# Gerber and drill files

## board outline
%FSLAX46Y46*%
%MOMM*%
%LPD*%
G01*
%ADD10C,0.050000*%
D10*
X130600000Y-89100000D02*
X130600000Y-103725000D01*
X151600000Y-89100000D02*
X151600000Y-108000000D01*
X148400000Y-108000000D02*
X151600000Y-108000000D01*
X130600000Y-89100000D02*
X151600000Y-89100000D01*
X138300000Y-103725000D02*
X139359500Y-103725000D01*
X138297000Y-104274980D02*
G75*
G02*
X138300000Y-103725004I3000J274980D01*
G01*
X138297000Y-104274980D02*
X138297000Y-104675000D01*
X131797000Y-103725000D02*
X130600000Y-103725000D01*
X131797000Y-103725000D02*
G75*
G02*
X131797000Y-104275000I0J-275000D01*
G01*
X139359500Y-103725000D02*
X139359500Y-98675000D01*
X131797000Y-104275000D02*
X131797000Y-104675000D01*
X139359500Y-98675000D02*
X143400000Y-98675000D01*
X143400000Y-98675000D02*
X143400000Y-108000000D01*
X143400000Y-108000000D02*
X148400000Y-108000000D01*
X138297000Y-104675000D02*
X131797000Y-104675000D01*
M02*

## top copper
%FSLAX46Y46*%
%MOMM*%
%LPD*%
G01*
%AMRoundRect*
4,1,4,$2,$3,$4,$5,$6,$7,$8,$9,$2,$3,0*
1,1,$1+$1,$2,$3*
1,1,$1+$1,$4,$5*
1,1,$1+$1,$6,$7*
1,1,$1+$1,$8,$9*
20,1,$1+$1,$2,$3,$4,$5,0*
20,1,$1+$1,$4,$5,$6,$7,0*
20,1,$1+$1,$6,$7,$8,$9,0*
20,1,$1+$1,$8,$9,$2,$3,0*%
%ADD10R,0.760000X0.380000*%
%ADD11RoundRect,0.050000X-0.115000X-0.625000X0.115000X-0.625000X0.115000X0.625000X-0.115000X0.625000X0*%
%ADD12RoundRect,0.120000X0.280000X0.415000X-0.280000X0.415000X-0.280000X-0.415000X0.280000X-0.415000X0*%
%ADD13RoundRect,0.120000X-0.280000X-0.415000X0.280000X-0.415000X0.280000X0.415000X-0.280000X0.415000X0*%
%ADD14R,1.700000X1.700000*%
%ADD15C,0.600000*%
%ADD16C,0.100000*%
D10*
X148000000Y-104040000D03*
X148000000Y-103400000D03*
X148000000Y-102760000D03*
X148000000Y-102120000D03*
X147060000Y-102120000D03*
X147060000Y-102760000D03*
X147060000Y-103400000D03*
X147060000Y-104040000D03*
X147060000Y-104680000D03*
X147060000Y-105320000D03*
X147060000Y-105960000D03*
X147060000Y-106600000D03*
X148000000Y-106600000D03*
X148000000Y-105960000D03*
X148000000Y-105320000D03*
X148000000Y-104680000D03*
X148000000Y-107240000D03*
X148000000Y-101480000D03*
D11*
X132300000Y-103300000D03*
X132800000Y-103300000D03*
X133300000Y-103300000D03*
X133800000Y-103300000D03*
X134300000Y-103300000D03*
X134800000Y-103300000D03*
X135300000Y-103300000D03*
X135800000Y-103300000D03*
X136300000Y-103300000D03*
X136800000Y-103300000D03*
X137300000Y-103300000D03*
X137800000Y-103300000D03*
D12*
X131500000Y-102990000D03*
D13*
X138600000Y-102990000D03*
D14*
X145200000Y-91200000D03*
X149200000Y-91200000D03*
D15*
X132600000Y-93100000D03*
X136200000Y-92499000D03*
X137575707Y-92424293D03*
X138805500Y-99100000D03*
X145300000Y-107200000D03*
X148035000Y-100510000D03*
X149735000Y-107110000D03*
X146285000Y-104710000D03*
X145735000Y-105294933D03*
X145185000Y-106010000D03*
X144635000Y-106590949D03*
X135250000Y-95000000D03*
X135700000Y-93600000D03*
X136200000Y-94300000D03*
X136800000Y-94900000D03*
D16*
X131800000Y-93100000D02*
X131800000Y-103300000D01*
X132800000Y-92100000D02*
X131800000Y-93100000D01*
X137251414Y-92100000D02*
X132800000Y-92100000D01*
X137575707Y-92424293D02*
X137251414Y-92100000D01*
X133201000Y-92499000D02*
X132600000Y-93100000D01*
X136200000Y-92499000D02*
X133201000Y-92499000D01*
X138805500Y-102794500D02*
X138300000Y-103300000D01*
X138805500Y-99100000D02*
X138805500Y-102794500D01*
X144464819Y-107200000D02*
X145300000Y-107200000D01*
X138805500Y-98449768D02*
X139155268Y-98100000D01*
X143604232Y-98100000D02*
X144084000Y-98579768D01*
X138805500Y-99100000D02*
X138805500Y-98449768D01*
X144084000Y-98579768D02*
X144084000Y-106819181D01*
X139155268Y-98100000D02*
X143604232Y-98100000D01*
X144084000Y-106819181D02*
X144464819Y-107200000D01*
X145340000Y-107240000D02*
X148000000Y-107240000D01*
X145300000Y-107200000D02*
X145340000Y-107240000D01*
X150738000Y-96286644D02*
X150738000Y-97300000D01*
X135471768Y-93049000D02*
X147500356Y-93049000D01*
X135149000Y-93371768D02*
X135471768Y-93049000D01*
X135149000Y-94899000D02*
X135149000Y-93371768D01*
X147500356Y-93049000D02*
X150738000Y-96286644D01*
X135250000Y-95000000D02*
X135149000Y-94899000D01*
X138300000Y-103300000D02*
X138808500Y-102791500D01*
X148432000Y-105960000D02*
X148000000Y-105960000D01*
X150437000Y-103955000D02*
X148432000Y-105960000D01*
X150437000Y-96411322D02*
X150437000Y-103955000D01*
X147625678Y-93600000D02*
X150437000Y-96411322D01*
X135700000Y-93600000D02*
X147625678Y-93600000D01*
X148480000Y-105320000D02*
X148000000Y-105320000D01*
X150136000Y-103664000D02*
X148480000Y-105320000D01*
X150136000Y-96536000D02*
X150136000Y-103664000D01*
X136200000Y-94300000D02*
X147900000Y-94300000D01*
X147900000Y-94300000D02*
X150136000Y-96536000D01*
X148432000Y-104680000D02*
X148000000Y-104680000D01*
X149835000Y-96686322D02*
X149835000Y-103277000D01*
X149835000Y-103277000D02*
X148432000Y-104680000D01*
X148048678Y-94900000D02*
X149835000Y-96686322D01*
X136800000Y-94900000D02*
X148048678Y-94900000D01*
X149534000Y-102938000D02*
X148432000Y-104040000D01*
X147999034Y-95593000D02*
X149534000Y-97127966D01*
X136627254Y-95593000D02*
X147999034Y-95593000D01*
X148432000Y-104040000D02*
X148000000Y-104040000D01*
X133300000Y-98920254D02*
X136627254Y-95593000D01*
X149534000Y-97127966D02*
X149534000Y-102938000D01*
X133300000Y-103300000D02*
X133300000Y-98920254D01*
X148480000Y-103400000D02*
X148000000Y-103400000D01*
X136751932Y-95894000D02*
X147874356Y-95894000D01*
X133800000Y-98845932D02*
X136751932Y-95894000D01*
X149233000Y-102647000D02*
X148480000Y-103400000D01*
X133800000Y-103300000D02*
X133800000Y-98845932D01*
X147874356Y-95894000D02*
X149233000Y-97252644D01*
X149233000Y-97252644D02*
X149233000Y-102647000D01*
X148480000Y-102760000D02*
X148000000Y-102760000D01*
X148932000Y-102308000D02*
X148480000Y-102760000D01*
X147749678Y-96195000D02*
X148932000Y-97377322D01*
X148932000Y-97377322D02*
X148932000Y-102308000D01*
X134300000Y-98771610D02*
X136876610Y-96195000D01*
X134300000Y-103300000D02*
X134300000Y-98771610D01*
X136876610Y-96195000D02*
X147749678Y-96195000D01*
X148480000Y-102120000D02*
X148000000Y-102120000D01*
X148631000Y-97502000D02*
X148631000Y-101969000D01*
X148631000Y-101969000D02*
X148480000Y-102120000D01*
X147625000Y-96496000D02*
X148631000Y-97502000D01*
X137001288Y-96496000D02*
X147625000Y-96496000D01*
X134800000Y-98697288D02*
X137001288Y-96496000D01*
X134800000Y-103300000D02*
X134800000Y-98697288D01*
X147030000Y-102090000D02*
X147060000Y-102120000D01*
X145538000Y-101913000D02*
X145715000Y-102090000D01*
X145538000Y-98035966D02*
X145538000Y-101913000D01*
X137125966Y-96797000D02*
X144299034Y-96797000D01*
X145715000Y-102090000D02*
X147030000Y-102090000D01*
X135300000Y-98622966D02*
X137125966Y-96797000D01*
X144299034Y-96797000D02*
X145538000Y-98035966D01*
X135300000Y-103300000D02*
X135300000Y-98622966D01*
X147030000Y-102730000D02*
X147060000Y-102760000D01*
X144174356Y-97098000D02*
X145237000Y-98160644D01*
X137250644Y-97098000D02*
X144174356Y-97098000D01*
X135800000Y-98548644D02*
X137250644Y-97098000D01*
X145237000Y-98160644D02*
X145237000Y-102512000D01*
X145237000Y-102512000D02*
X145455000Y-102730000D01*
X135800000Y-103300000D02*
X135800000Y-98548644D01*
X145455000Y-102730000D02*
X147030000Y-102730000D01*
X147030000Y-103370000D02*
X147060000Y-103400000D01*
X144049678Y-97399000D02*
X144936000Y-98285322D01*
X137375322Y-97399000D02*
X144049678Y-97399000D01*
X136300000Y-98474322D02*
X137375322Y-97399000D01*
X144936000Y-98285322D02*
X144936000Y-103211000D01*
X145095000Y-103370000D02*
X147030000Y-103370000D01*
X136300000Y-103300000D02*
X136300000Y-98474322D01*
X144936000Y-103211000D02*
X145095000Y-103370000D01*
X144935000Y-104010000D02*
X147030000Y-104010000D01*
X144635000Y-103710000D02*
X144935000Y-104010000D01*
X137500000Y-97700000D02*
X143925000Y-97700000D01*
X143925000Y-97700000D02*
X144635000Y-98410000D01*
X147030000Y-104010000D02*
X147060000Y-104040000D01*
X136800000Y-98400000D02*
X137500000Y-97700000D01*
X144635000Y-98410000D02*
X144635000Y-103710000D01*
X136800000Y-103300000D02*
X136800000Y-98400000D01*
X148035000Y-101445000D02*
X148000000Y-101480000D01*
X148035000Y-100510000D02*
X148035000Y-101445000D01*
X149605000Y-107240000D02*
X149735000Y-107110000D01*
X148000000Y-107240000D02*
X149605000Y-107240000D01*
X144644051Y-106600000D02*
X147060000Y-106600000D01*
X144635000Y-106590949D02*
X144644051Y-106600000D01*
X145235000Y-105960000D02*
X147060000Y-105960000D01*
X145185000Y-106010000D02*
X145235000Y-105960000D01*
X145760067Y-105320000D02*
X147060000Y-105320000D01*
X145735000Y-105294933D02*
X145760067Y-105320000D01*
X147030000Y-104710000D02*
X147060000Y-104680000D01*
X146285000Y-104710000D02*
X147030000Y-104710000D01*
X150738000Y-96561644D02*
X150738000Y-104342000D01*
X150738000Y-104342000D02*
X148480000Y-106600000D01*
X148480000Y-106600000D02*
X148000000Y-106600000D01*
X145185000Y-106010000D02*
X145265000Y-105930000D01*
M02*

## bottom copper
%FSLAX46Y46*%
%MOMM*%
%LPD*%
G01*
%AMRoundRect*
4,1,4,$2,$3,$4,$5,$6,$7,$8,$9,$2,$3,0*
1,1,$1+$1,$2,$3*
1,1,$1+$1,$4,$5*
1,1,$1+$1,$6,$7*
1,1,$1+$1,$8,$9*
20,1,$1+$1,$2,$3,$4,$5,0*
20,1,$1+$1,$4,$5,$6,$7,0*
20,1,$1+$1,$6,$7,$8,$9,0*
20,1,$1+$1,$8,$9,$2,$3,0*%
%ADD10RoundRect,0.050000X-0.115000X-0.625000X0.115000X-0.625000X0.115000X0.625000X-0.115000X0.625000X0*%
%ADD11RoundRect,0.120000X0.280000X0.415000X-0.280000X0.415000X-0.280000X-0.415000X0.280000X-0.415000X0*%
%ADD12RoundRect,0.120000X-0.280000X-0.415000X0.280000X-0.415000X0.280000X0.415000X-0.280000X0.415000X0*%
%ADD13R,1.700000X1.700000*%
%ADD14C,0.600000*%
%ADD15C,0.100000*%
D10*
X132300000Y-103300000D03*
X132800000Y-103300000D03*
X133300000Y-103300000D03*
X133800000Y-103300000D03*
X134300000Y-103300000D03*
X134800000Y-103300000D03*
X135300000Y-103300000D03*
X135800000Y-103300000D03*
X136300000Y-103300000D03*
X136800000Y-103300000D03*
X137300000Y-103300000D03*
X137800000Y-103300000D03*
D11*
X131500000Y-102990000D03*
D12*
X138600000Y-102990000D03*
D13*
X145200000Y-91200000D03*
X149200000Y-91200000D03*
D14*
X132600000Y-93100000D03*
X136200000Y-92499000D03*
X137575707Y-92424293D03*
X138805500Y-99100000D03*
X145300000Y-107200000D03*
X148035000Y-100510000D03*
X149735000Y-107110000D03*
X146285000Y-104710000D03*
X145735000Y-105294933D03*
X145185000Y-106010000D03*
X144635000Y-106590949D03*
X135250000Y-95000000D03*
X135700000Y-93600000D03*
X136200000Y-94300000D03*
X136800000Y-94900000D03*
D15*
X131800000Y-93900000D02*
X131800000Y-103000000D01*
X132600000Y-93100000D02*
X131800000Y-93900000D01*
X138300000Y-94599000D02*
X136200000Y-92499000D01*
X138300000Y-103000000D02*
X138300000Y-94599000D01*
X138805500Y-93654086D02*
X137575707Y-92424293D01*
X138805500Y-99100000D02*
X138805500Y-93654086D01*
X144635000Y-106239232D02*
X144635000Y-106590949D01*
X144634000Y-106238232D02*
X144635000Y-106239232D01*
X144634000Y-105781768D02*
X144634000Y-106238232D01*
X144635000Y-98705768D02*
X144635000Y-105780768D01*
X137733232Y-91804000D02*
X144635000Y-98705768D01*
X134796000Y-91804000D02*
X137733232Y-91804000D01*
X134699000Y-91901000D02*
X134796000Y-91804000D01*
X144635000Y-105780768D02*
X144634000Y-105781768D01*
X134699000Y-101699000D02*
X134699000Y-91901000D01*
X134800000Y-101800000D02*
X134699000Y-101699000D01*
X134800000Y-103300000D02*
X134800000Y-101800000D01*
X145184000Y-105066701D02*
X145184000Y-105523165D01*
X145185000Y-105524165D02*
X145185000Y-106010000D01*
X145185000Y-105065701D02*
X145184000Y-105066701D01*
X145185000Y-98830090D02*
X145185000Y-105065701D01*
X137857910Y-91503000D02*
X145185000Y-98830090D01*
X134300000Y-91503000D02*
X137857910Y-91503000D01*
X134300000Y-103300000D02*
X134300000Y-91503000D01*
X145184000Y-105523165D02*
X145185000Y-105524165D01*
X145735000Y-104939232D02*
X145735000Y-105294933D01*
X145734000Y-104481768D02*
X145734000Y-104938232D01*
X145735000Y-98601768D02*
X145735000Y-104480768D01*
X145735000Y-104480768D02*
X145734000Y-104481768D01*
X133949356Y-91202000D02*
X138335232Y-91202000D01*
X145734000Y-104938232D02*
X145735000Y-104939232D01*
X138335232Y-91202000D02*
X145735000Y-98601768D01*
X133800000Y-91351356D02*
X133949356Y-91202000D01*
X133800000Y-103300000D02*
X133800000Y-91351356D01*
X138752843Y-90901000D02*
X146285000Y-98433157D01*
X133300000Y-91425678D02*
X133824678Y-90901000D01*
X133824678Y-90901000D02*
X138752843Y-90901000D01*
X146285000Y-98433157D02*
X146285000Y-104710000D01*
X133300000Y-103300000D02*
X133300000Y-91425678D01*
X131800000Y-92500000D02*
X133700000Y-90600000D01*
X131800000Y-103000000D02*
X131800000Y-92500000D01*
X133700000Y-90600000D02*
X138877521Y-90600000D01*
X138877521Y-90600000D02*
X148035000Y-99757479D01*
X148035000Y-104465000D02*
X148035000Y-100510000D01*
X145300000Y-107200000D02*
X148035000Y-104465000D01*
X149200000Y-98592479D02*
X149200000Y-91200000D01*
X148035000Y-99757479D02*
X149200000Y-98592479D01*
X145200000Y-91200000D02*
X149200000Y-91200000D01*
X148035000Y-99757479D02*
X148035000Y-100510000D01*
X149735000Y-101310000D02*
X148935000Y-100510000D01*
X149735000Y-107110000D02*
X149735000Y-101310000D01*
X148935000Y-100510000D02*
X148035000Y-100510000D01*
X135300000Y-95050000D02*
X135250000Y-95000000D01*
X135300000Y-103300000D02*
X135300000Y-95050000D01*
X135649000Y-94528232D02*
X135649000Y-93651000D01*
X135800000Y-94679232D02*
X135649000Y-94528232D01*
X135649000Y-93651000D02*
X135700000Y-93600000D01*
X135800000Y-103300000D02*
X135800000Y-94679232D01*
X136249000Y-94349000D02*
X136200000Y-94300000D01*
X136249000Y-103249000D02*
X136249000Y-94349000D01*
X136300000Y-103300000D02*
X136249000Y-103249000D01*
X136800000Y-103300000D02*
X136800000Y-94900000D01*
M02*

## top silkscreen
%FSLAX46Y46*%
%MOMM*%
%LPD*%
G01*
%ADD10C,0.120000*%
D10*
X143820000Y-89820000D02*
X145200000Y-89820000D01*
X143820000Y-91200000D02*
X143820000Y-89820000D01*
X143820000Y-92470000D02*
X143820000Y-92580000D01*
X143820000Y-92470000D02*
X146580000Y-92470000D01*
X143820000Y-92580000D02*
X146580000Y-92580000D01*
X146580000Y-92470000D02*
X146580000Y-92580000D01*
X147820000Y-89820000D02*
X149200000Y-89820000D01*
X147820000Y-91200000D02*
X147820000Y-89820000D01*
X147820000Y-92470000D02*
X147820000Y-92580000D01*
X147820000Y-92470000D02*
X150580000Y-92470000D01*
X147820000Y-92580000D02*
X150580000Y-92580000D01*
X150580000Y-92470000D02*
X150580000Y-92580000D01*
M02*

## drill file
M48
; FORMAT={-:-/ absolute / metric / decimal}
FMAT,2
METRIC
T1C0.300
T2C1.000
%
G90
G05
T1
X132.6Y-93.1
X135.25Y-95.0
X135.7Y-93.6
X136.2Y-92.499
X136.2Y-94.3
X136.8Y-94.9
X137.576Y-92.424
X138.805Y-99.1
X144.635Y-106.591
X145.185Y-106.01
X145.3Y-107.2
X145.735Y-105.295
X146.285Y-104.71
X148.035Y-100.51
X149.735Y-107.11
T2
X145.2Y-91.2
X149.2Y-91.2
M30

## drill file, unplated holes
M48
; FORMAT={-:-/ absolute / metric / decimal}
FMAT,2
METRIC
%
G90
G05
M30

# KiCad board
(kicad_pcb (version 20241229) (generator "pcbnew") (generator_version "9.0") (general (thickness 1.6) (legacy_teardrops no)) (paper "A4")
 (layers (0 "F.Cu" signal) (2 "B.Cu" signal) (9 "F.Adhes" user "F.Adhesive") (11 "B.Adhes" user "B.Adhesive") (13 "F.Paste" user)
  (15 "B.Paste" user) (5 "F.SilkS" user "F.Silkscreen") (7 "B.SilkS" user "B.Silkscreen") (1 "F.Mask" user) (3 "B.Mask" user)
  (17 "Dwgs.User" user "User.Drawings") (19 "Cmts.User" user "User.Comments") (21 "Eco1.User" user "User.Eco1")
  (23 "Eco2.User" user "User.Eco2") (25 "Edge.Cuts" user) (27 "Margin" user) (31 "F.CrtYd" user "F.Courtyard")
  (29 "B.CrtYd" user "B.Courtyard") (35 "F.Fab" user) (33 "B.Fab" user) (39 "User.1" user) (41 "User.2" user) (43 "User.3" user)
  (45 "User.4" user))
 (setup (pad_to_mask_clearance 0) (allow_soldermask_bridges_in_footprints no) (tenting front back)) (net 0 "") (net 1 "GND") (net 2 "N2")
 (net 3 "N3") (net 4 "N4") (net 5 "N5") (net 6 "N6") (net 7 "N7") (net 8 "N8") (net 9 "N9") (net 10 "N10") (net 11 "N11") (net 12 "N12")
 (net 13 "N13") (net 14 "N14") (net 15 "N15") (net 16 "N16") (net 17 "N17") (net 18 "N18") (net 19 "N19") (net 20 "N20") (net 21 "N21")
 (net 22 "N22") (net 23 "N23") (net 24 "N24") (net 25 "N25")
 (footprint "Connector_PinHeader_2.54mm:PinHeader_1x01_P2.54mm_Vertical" (layer "F.Cu") (at 149.2 91.2)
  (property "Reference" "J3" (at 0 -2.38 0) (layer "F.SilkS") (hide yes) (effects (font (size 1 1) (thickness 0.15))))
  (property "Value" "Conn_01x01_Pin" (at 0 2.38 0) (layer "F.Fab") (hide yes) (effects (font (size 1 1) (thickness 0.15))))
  (fp_line (start -1.38 -1.38) (end 0 -1.38) (stroke (width 0.12) (type solid)) (layer "F.SilkS"))
  (fp_line (start -1.38 0) (end -1.38 -1.38) (stroke (width 0.12) (type solid)) (layer "F.SilkS"))
  (fp_line (start -1.38 1.27) (end -1.38 1.38) (stroke (width 0.12) (type solid)) (layer "F.SilkS"))
  (fp_line (start -1.38 1.27) (end 1.38 1.27) (stroke (width 0.12) (type solid)) (layer "F.SilkS"))
  (fp_line (start -1.38 1.38) (end 1.38 1.38) (stroke (width 0.12) (type solid)) (layer "F.SilkS"))
  (fp_line (start 1.38 1.27) (end 1.38 1.38) (stroke (width 0.12) (type solid)) (layer "F.SilkS"))
  (pad "1" thru_hole rect (at 0 0) (size 1.7 1.7) (drill 1) (layers "*.Cu" "*.Mask") (remove_unused_layers no) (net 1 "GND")))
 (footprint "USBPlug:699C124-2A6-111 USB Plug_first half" (layer "F.Cu") (at 134.8 100.3)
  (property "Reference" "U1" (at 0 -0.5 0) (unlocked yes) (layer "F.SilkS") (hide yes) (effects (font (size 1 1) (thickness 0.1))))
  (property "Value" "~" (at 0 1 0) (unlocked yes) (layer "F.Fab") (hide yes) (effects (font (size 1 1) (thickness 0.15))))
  (pad "0" smd roundrect (at -2.5 3) (size 0.33 1.35) (layers "F.Cu" "F.Mask" "F.Paste") (roundrect_rratio 0.1515151515) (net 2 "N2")
   (thermal_bridge_angle 45))
  (pad "1" smd roundrect (at -2 3) (size 0.33 1.35) (layers "F.Cu" "F.Mask" "F.Paste") (roundrect_rratio 0.1515151515) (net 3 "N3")
   (thermal_bridge_angle 45))
  (pad "2" smd roundrect (at -1.5 3) (size 0.33 1.35) (layers "F.Cu" "F.Mask" "F.Paste") (roundrect_rratio 0.1515151515) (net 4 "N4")
   (thermal_bridge_angle 45))
  (pad "3" smd roundrect (at -1 3) (size 0.33 1.35) (layers "F.Cu" "F.Mask" "F.Paste") (roundrect_rratio 0.1515151515) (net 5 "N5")
   (thermal_bridge_angle 45))
  (pad "4" smd roundrect (at -0.5 3) (size 0.33 1.35) (layers "F.Cu" "F.Mask" "F.Paste") (roundrect_rratio 0.1515151515) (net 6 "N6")
   (thermal_bridge_angle 45))
  (pad "5" smd roundrect (at 0 3) (size 0.33 1.35) (layers "F.Cu" "F.Mask" "F.Paste") (roundrect_rratio 0.1515151515) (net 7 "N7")
   (thermal_bridge_angle 45))
  (pad "6" smd roundrect (at 0.5 3) (size 0.33 1.35) (layers "F.Cu" "F.Mask" "F.Paste") (roundrect_rratio 0.1515151515) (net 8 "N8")
   (thermal_bridge_angle 45))
  (pad "7" smd roundrect (at 1 3) (size 0.33 1.35) (layers "F.Cu" "F.Mask" "F.Paste") (roundrect_rratio 0.1515151515) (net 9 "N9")
   (thermal_bridge_angle 45))
  (pad "8" smd roundrect (at 1.5 3) (size 0.33 1.35) (layers "F.Cu" "F.Mask" "F.Paste") (roundrect_rratio 0.1515151515) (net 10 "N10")
   (thermal_bridge_angle 45))
  (pad "9" smd roundrect (at 2 3) (size 0.33 1.35) (layers "F.Cu" "F.Mask" "F.Paste") (roundrect_rratio 0.1515151515) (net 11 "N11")
   (thermal_bridge_angle 45))
  (pad "10" smd roundrect (at 2.5 3) (size 0.33 1.35) (layers "F.Cu" "F.Mask" "F.Paste") (roundrect_rratio 0.1515151515) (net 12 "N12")
   (thermal_bridge_angle 45))
  (pad "11" smd roundrect (at 3 3) (size 0.33 1.35) (layers "F.Cu" "F.Mask" "F.Paste") (roundrect_rratio 0.1515151515) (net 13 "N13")
   (thermal_bridge_angle 45))
  (pad "24" smd roundrect (at -3 3 180) (size 0.8 1.07) (drill (offset 0.3 0.31)) (layers "F.Cu" "F.Mask" "F.Paste") (roundrect_rratio 0.15)
   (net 1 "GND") (thermal_bridge_angle 45))
  (pad "25" smd roundrect (at 3.5 3) (size 0.8 1.07) (drill (offset 0.3 -0.31)) (layers "F.Cu" "F.Mask" "F.Paste") (roundrect_rratio 0.15)
   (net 1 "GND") (thermal_bridge_angle 45)))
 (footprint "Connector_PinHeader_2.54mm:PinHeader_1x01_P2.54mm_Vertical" (layer "F.Cu") (at 145.2 91.2)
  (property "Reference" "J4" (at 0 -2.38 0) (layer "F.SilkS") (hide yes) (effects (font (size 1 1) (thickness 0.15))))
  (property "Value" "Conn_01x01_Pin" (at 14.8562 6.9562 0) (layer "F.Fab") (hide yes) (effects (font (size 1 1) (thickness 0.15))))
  (fp_line (start -1.38 -1.38) (end 0 -1.38) (stroke (width 0.12) (type solid)) (layer "F.SilkS"))
  (fp_line (start -1.38 0) (end -1.38 -1.38) (stroke (width 0.12) (type solid)) (layer "F.SilkS"))
  (fp_line (start -1.38 1.27) (end -1.38 1.38) (stroke (width 0.12) (type solid)) (layer "F.SilkS"))
  (fp_line (start -1.38 1.27) (end 1.38 1.27) (stroke (width 0.12) (type solid)) (layer "F.SilkS"))
  (fp_line (start -1.38 1.38) (end 1.38 1.38) (stroke (width 0.12) (type solid)) (layer "F.SilkS"))
  (fp_line (start 1.38 1.27) (end 1.38 1.38) (stroke (width 0.12) (type solid)) (layer "F.SilkS"))
  (pad "1" thru_hole rect (at 0 0) (size 1.7 1.7) (drill 1) (layers "*.Cu" "*.Mask") (remove_unused_layers no) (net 1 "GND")))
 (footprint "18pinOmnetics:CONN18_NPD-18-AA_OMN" (layer "F.Cu") (at 148.94 104.04 90)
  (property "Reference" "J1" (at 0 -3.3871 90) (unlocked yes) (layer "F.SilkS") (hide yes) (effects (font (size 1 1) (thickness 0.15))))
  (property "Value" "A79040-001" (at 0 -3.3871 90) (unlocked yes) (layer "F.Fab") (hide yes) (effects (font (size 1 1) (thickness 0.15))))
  (pad "0" smd rect (at 0 -0.94 90) (size 0.38 0.76) (layers "F.Cu" "F.Mask" "F.Paste") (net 4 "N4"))
  (pad "1" smd rect (at 0.64 -0.94 90) (size 0.38 0.76) (layers "F.Cu" "F.Mask" "F.Paste") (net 5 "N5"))
  (pad "2" smd rect (at 1.28 -0.94 90) (size 0.38 0.76) (layers "F.Cu" "F.Mask" "F.Paste") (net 6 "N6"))
  (pad "3" smd rect (at 1.92 -0.94 90) (size 0.38 0.76) (layers "F.Cu" "F.Mask" "F.Paste") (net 7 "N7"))
  (pad "4" smd rect (at 1.92 -1.88 90) (size 0.38 0.76) (layers "F.Cu" "F.Mask" "F.Paste") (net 8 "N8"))
  (pad "5" smd rect (at 1.28 -1.88 90) (size 0.38 0.76) (layers "F.Cu" "F.Mask" "F.Paste") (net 9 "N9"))
  (pad "6" smd rect (at 0.64 -1.88 90) (size 0.38 0.76) (layers "F.Cu" "F.Mask" "F.Paste") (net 10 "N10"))
  (pad "7" smd rect (at 0 -1.88 90) (size 0.38 0.76) (layers "F.Cu" "F.Mask" "F.Paste") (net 11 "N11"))
  (pad "8" smd rect (at -0.64 -1.88 90) (size 0.38 0.76) (layers "F.Cu" "F.Mask" "F.Paste") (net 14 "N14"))
  (pad "9" smd rect (at -1.28 -1.88 90) (size 0.38 0.76) (layers "F.Cu" "F.Mask" "F.Paste") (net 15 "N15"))
  (pad "10" smd rect (at -1.92 -1.88 90) (size 0.38 0.76) (layers "F.Cu" "F.Mask" "F.Paste") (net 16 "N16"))
  (pad "11" smd rect (at -2.56 -1.88 90) (size 0.38 0.76) (layers "F.Cu" "F.Mask" "F.Paste") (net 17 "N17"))
  (pad "12" smd rect (at -2.56 -0.94 90) (size 0.38 0.76) (layers "F.Cu" "F.Mask" "F.Paste") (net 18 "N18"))
  (pad "13" smd rect (at -1.92 -0.94 90) (size 0.38 0.76) (layers "F.Cu" "F.Mask" "F.Paste") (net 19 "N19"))
  (pad "14" smd rect (at -1.28 -0.94 90) (size 0.38 0.76) (layers "F.Cu" "F.Mask" "F.Paste") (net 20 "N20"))
  (pad "15" smd rect (at -0.64 -0.94 90) (size 0.38 0.76) (layers "F.Cu" "F.Mask" "F.Paste") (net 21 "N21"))
  (pad "16" smd rect (at -3.2 -0.94 90) (size 0.38 0.76) (layers "F.Cu" "F.Mask" "F.Paste") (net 1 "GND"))
  (pad "17" smd rect (at 2.56 -0.94 90) (size 0.38 0.76) (layers "F.Cu" "F.Mask" "F.Paste") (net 1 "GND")))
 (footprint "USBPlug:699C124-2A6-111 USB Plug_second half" (layer "B.Cu") (at 134.8 106.3)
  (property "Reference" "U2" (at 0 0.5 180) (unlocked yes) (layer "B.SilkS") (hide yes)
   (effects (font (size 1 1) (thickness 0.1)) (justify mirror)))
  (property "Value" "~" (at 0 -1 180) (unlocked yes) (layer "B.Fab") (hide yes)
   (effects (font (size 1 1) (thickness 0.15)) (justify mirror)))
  (pad "12" smd roundrect (at -2.5 -3) (size 0.33 1.35) (layers "B.Cu" "B.Mask" "B.Paste") (roundrect_rratio 0.1515151515) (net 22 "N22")
   (thermal_bridge_angle 45))
  (pad "13" smd roundrect (at -2 -3) (size 0.33 1.35) (layers "B.Cu" "B.Mask" "B.Paste") (roundrect_rratio 0.1515151515) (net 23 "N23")
   (thermal_bridge_angle 45))
  (pad "14" smd roundrect (at -1.5 -3) (size 0.33 1.35) (layers "B.Cu" "B.Mask" "B.Paste") (roundrect_rratio 0.1515151515) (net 14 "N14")
   (thermal_bridge_angle 45))
  (pad "15" smd roundrect (at -1 -3) (size 0.33 1.35) (layers "B.Cu" "B.Mask" "B.Paste") (roundrect_rratio 0.1515151515) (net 15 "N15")
   (thermal_bridge_angle 45))
  (pad "16" smd roundrect (at -0.5 -3) (size 0.33 1.35) (layers "B.Cu" "B.Mask" "B.Paste") (roundrect_rratio 0.1515151515) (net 16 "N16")
   (thermal_bridge_angle 45))
  (pad "17" smd roundrect (at 0 -3) (size 0.33 1.35) (layers "B.Cu" "B.Mask" "B.Paste") (roundrect_rratio 0.1515151515) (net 17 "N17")
   (thermal_bridge_angle 45))
  (pad "18" smd roundrect (at 0.5 -3) (size 0.33 1.35) (layers "B.Cu" "B.Mask" "B.Paste") (roundrect_rratio 0.1515151515) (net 18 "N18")
   (thermal_bridge_angle 45))
  (pad "19" smd roundrect (at 1 -3) (size 0.33 1.35) (layers "B.Cu" "B.Mask" "B.Paste") (roundrect_rratio 0.1515151515) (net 19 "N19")
   (thermal_bridge_angle 45))
  (pad "20" smd roundrect (at 1.5 -3) (size 0.33 1.35) (layers "B.Cu" "B.Mask" "B.Paste") (roundrect_rratio 0.1515151515) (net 20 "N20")
   (thermal_bridge_angle 45))
  (pad "21" smd roundrect (at 2 -3) (size 0.33 1.35) (layers "B.Cu" "B.Mask" "B.Paste") (roundrect_rratio 0.1515151515) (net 21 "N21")
   (thermal_bridge_angle 45))
  (pad "22" smd roundrect (at 2.5 -3) (size 0.33 1.35) (layers "B.Cu" "B.Mask" "B.Paste") (roundrect_rratio 0.1515151515) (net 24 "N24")
   (thermal_bridge_angle 45))
  (pad "23" smd roundrect (at 3 -3) (size 0.33 1.35) (layers "B.Cu" "B.Mask" "B.Paste") (roundrect_rratio 0.1515151515) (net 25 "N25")
   (thermal_bridge_angle 45))
  (pad "26" smd roundrect (at -3 -3.3 180) (size 0.8 1.07) (drill (offset 0.3 0.01)) (layers "B.Cu" "B.Mask" "B.Paste")
   (roundrect_rratio 0.15) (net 1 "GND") (thermal_bridge_angle 45))
  (pad "27" smd roundrect (at 3.5 -3.3) (size 0.8 1.07) (drill (offset 0.3 -0.01)) (layers "B.Cu" "B.Mask" "B.Paste")
   (roundrect_rratio 0.15) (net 1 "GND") (thermal_bridge_angle 45)))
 (gr_arc (start 138.297 104.27498) (mid 138.025 104) (end 138.3 103.725) (stroke (width 0.05) (type default)) (layer "Edge.Cuts"))
 (gr_line (start 130.6 89.1) (end 151.6 89.1) (stroke (width 0.05) (type default)) (layer "Edge.Cuts"))
 (gr_line (start 143.4 98.675) (end 143.4 108) (stroke (width 0.05) (type default)) (layer "Edge.Cuts"))
 (gr_line (start 139.3595 103.725) (end 139.3595 98.675) (stroke (width 0.05) (type default)) (layer "Edge.Cuts"))
 (gr_line (start 138.3 103.725) (end 139.3595 103.725) (stroke (width 0.05) (type default)) (layer "Edge.Cuts"))
 (gr_line (start 139.3595 98.675) (end 143.4 98.675) (stroke (width 0.05) (type default)) (layer "Edge.Cuts"))
 (gr_line (start 143.4 108) (end 148.4 108) (stroke (width 0.05) (type default)) (layer "Edge.Cuts"))
 (gr_line (start 131.797 104.275) (end 131.797 104.675) (stroke (width 0.05) (type default)) (layer "Edge.Cuts"))
 (gr_line (start 138.297 104.27498) (end 138.297 104.675) (stroke (width 0.05) (type default)) (layer "Edge.Cuts"))
 (gr_arc (start 131.797 103.725) (mid 132.072 104) (end 131.797 104.275) (stroke (width 0.05) (type default)) (layer "Edge.Cuts"))
 (gr_line (start 151.6 89.1) (end 151.6 108) (stroke (width 0.05) (type default)) (layer "Edge.Cuts"))
 (gr_line (start 148.4 108) (end 151.6 108) (stroke (width 0.05) (type default)) (layer "Edge.Cuts"))
 (gr_line (start 138.297 104.675) (end 131.797 104.675) (stroke (width 0.05) (type default)) (layer "Edge.Cuts"))
 (gr_line (start 130.6 89.1) (end 130.6 103.725) (stroke (width 0.05) (type default)) (layer "Edge.Cuts"))
 (gr_line (start 131.797 103.725) (end 130.6 103.725) (stroke (width 0.05) (type default)) (layer "Edge.Cuts"))
 (segment (start 148.035 101.445) (end 148 101.48) (width 0.1) (layer "F.Cu") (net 1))
 (segment (start 139.155268 98.1) (end 143.604232 98.1) (width 0.1) (layer "F.Cu") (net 1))
 (segment (start 144.084 98.579768) (end 144.084 106.819181) (width 0.1) (layer "F.Cu") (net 1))
 (segment (start 138.8055 99.1) (end 138.8055 102.7945) (width 0.1) (layer "F.Cu") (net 1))
 (segment (start 136.2 92.499) (end 133.201 92.499) (width 0.1) (layer "F.Cu") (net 1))
 (segment (start 137.251414 92.1) (end 132.8 92.1) (width 0.1) (layer "F.Cu") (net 1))
 (segment (start 138.3 103.3) (end 138.8085 102.7915) (width 0.1) (layer "F.Cu") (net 1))
 (segment (start 148 107.24) (end 149.605 107.24) (width 0.1) (layer "F.Cu") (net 1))
 (segment (start 149.605 107.24) (end 149.735 107.11) (width 0.1) (layer "F.Cu") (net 1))
 (segment (start 132.8 92.1) (end 131.8 93.1) (width 0.1) (layer "F.Cu") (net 1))
 (segment (start 145.34 107.24) (end 148 107.24) (width 0.1) (layer "F.Cu") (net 1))
 (segment (start 145.3 107.2) (end 145.34 107.24) (width 0.1) (layer "F.Cu") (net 1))
 (segment (start 144.464819 107.2) (end 145.3 107.2) (width 0.1) (layer "F.Cu") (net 1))
 (segment (start 143.604232 98.1) (end 144.084 98.579768) (width 0.1) (layer "F.Cu") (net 1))
 (segment (start 144.084 106.819181) (end 144.464819 107.2) (width 0.1) (layer "F.Cu") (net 1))
 (segment (start 133.201 92.499) (end 132.6 93.1) (width 0.1) (layer "F.Cu") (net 1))
 (segment (start 138.8055 98.449768) (end 139.155268 98.1) (width 0.1) (layer "F.Cu") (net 1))
 (segment (start 138.8055 99.1) (end 138.8055 98.449768) (width 0.1) (layer "F.Cu") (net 1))
 (segment (start 137.575707 92.424293) (end 137.251414 92.1) (width 0.1) (layer "F.Cu") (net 1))
 (segment (start 131.8 93.1) (end 131.8 103.3) (width 0.1) (layer "F.Cu") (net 1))
 (segment (start 138.8055 102.7945) (end 138.3 103.3) (width 0.1) (layer "F.Cu") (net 1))
 (segment (start 148.035 100.51) (end 148.035 101.445) (width 0.1) (layer "F.Cu") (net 1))
 (via (at 149.735 107.11) (size 0.6) (drill 0.3) (layers "F.Cu" "B.Cu") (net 1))
 (via (at 136.2 92.499) (size 0.6) (drill 0.3) (layers "F.Cu" "B.Cu") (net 1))
 (via (at 137.575707 92.424293) (size 0.6) (drill 0.3) (layers "F.Cu" "B.Cu") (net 1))
 (via (at 138.8055 99.1) (size 0.6) (drill 0.3) (layers "F.Cu" "B.Cu") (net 1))
 (via (at 132.6 93.1) (size 0.6) (drill 0.3) (layers "F.Cu" "B.Cu") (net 1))
 (via (at 145.3 107.2) (size 0.6) (drill 0.3) (layers "F.Cu" "B.Cu") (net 1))
 (via (at 148.035 100.51) (size 0.6) (drill 0.3) (layers "F.Cu" "B.Cu") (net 1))
 (segment (start 148.035 99.757479) (end 148.035 100.51) (width 0.1) (layer "B.Cu") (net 1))
 (segment (start 145.2 91.2) (end 149.2 91.2) (width 0.1) (layer "B.Cu") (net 1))
 (segment (start 149.735 107.11) (end 149.735 101.31) (width 0.1) (layer "B.Cu") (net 1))
 (segment (start 148.035 99.757479) (end 149.2 98.592479) (width 0.1) (layer "B.Cu") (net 1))
 (segment (start 133.7 90.6) (end 138.877521 90.6) (width 0.1) (layer "B.Cu") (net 1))
 (segment (start 149.2 98.592479) (end 149.2 91.2) (width 0.1) (layer "B.Cu") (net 1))
 (segment (start 132.6 93.1) (end 131.8 93.9) (width 0.1) (layer "B.Cu") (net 1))
 (segment (start 148.935 100.51) (end 148.035 100.51) (width 0.1) (layer "B.Cu") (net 1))
 (segment (start 131.8 93.9) (end 131.8 103) (width 0.1) (layer "B.Cu") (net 1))
 (segment (start 138.877521 90.6) (end 148.035 99.757479) (width 0.1) (layer "B.Cu") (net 1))
 (segment (start 138.3 94.599) (end 136.2 92.499) (width 0.1) (layer "B.Cu") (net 1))
 (segment (start 138.8055 99.1) (end 138.8055 93.654086) (width 0.1) (layer "B.Cu") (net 1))
 (segment (start 138.8055 93.654086) (end 137.575707 92.424293) (width 0.1) (layer "B.Cu") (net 1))
 (segment (start 131.8 92.5) (end 133.7 90.6) (width 0.1) (layer "B.Cu") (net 1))
 (segment (start 148.035 104.465) (end 148.035 100.51) (width 0.1) (layer "B.Cu") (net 1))
 (segment (start 145.3 107.2) (end 148.035 104.465) (width 0.1) (layer "B.Cu") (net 1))
 (segment (start 138.3 103) (end 138.3 94.599) (width 0.1) (layer "B.Cu") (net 1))
 (segment (start 149.735 101.31) (end 148.935 100.51) (width 0.1) (layer "B.Cu") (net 1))
 (segment (start 131.8 103) (end 131.8 92.5) (width 0.1) (layer "B.Cu") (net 1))
 (segment (start 145.538 101.913) (end 145.715 102.09) (width 0.1) (layer "F.Cu") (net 8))
 (segment (start 144.299034 96.797) (end 145.538 98.035966) (width 0.1) (layer "F.Cu") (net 8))
 (segment (start 137.125966 96.797) (end 144.299034 96.797) (width 0.1) (layer "F.Cu") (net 8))
 (segment (start 145.715 102.09) (end 147.03 102.09) (width 0.1) (layer "F.Cu") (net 8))
 (segment (start 135.3 103.3) (end 135.3 98.622966) (width 0.1) (layer "F.Cu") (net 8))
 (segment (start 147.03 102.09) (end 147.06 102.12) (width 0.1) (layer "F.Cu") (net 8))
 (segment (start 135.3 98.622966) (end 137.125966 96.797) (width 0.1) (layer "F.Cu") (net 8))
 (segment (start 145.538 98.035966) (end 145.538 101.913) (width 0.1) (layer "F.Cu") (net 8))
 (segment (start 144.635 106.590949) (end 144.644051 106.6) (width 0.1) (layer "F.Cu") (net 17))
 (segment (start 144.644051 106.6) (end 147.06 106.6) (width 0.1) (layer "F.Cu") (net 17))
 (via (at 144.635 106.590949) (size 0.6) (drill 0.3) (layers "F.Cu" "B.Cu") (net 17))
 (segment (start 144.635 105.780768) (end 144.634 105.781768) (width 0.1) (layer "B.Cu") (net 17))
 (segment (start 134.699 101.699) (end 134.699 91.901) (width 0.1) (layer "B.Cu") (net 17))
 (segment (start 144.634 105.781768) (end 144.634 106.238232) (width 0.1) (layer "B.Cu") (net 17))
 (segment (start 134.8 101.8) (end 134.699 101.699) (width 0.1) (layer "B.Cu") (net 17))
 (segment (start 144.634 106.238232) (end 144.635 106.239232) (width 0.1) (layer "B.Cu") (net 17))
 (segment (start 134.796 91.804) (end 137.733232 91.804) (width 0.1) (layer "B.Cu") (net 17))
 (segment (start 134.8 103.3) (end 134.8 101.8) (width 0.1) (layer "B.Cu") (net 17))
 (segment (start 144.635 98.705768) (end 144.635 105.780768) (width 0.1) (layer "B.Cu") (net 17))
 (segment (start 144.635 106.239232) (end 144.635 106.590949) (width 0.1) (layer "B.Cu") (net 17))
 (segment (start 134.699 91.901) (end 134.796 91.804) (width 0.1) (layer "B.Cu") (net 17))
 (segment (start 137.733232 91.804) (end 144.635 98.705768) (width 0.1) (layer "B.Cu") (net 17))
 (segment (start 144.936 98.285322) (end 144.936 103.211) (width 0.1) (layer "F.Cu") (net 10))
 (segment (start 136.3 98.474322) (end 137.375322 97.399) (width 0.1) (layer "F.Cu") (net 10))
 (segment (start 137.375322 97.399) (end 144.049678 97.399) (width 0.1) (layer "F.Cu") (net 10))
 (segment (start 145.095 103.37) (end 147.03 103.37) (width 0.1) (layer "F.Cu") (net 10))
 (segment (start 144.049678 97.399) (end 144.936 98.285322) (width 0.1) (layer "F.Cu") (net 10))
 (segment (start 144.936 103.211) (end 145.095 103.37) (width 0.1) (layer "F.Cu") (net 10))
 (segment (start 147.03 103.37) (end 147.06 103.4) (width 0.1) (layer "F.Cu") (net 10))
 (segment (start 136.3 103.3) (end 136.3 98.474322) (width 0.1) (layer "F.Cu") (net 10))
 (segment (start 145.735 105.294933) (end 145.760067 105.32) (width 0.1) (layer "F.Cu") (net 15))
 (segment (start 145.760067 105.32) (end 147.06 105.32) (width 0.1) (layer "F.Cu") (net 15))
 (via (at 145.735 105.294933) (size 0.6) (drill 0.3) (layers "F.Cu" "B.Cu") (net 15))
 (segment (start 145.735 104.480768) (end 145.734 104.481768) (width 0.1) (layer "B.Cu") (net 15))
 (segment (start 133.8 103.3) (end 133.8 91.351356) (width 0.1) (layer "B.Cu") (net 15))
 (segment (start 145.735 98.601768) (end 145.735 104.480768) (width 0.1) (layer "B.Cu") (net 15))
 (segment (start 133.949356 91.202) (end 138.335232 91.202) (width 0.1) (layer "B.Cu") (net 15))
 (segment (start 138.335232 91.202) (end 145.735 98.601768) (width 0.1) (layer "B.Cu") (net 15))
 (segment (start 145.734 104.938232) (end 145.735 104.939232) (width 0.1) (layer "B.Cu") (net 15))
 (segment (start 145.734 104.481768) (end 145.734 104.938232) (width 0.1) (layer "B.Cu") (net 15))
 (segment (start 145.735 104.939232) (end 145.735 105.294933) (width 0.1) (layer "B.Cu") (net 15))
 (segment (start 133.8 91.351356) (end 133.949356 91.202) (width 0.1) (layer "B.Cu") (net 15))
 (segment (start 136.2 94.3) (end 147.9 94.3) (width 0.1) (layer "F.Cu") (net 20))
 (segment (start 150.136 96.536) (end 150.136 103.664) (width 0.1) (layer "F.Cu") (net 20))
 (segment (start 147.9 94.3) (end 150.136 96.536) (width 0.1) (layer "F.Cu") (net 20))
 (segment (start 150.136 103.664) (end 148.48 105.32) (width 0.1) (layer "F.Cu") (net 20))
 (segment (start 148.48 105.32) (end 148 105.32) (width 0.1) (layer "F.Cu") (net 20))
 (via (at 136.2 94.3) (size 0.6) (drill 0.3) (layers "F.Cu" "B.Cu") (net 20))
 (segment (start 136.3 103.3) (end 136.249 103.249) (width 0.1) (layer "B.Cu") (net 20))
 (segment (start 136.249 94.349) (end 136.2 94.3) (width 0.1) (layer "B.Cu") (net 20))
 (segment (start 136.249 103.249) (end 136.249 94.349) (width 0.1) (layer "B.Cu") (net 20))
 (segment (start 149.534 102.938) (end 148.432 104.04) (width 0.1) (layer "F.Cu") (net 4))
 (segment (start 149.534 97.127966) (end 149.534 102.938) (width 0.1) (layer "F.Cu") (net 4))
 (segment (start 133.3 98.920254) (end 136.627254 95.593) (width 0.1) (layer "F.Cu") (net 4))
 (segment (start 136.627254 95.593) (end 147.999034 95.593) (width 0.1) (layer "F.Cu") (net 4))
 (segment (start 133.3 103.3) (end 133.3 98.920254) (width 0.1) (layer "F.Cu") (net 4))
 (segment (start 148.432 104.04) (end 148 104.04) (width 0.1) (layer "F.Cu") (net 4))
 (segment (start 147.999034 95.593) (end 149.534 97.127966) (width 0.1) (layer "F.Cu") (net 4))
 (segment (start 150.738 104.342) (end 148.48 106.6) (width 0.1) (layer "F.Cu") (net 18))
 (segment (start 135.25 95) (end 135.149 94.899) (width 0.1) (layer "F.Cu") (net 18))
 (segment (start 135.149 94.899) (end 135.149 93.371768) (width 0.1) (layer "F.Cu") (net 18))
 (segment (start 150.738 96.286644) (end 150.738 97.3) (width 0.1) (layer "F.Cu") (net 18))
 (segment (start 147.500356 93.049) (end 150.738 96.286644) (width 0.1) (layer "F.Cu") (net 18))
 (segment (start 150.738 96.561644) (end 150.738 104.342) (width 0.1) (layer "F.Cu") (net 18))
 (segment (start 135.149 93.371768) (end 135.471768 93.049) (width 0.1) (layer "F.Cu") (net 18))
 (segment (start 135.471768 93.049) (end 147.500356 93.049) (width 0.1) (layer "F.Cu") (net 18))
 (segment (start 148.48 106.6) (end 148 106.6) (width 0.1) (layer "F.Cu") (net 18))
 (via (at 135.25 95) (size 0.6) (drill 0.3) (layers "F.Cu" "B.Cu") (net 18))
 (segment (start 135.3 103.3) (end 135.3 95.05) (width 0.1) (layer "B.Cu") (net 18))
 (segment (start 135.3 95.05) (end 135.25 95) (width 0.1) (layer "B.Cu") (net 18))
 (segment (start 144.635 98.41) (end 144.635 103.71) (width 0.1) (layer "F.Cu") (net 11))
 (segment (start 144.635 103.71) (end 144.935 104.01) (width 0.1) (layer "F.Cu") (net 11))
 (segment (start 144.935 104.01) (end 147.03 104.01) (width 0.1) (layer "F.Cu") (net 11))
 (segment (start 136.8 98.4) (end 137.5 97.7) (width 0.1) (layer "F.Cu") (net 11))
 (segment (start 136.8 103.3) (end 136.8 98.4) (width 0.1) (layer "F.Cu") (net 11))
 (segment (start 137.5 97.7) (end 143.925 97.7) (width 0.1) (layer "F.Cu") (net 11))
 (segment (start 147.03 104.01) (end 147.06 104.04) (width 0.1) (layer "F.Cu") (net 11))
 (segment (start 143.925 97.7) (end 144.635 98.41) (width 0.1) (layer "F.Cu") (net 11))
 (segment (start 145.185 106.01) (end 145.235 105.96) (width 0.1) (layer "F.Cu") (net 16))
 (segment (start 145.185 106.01) (end 145.265 105.93) (width 0.1) (layer "F.Cu") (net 16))
 (segment (start 145.235 105.96) (end 147.06 105.96) (width 0.1) (layer "F.Cu") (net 16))
 (via (at 145.185 106.01) (size 0.6) (drill 0.3) (layers "F.Cu" "B.Cu") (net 16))
 (segment (start 145.184 105.523165) (end 145.185 105.524165) (width 0.1) (layer "B.Cu") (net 16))
 (segment (start 145.185 105.065701) (end 145.184 105.066701) (width 0.1) (layer "B.Cu") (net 16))
 (segment (start 134.3 91.503) (end 137.85791 91.503) (width 0.1) (layer "B.Cu") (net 16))
 (segment (start 145.185 98.83009) (end 145.185 105.065701) (width 0.1) (layer "B.Cu") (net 16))
 (segment (start 137.85791 91.503) (end 145.185 98.83009) (width 0.1) (layer "B.Cu") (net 16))
 (segment (start 145.184 105.066701) (end 145.184 105.523165) (width 0.1) (layer "B.Cu") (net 16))
 (segment (start 134.3 103.3) (end 134.3 91.503) (width 0.1) (layer "B.Cu") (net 16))
 (segment (start 145.185 105.524165) (end 145.185 106.01) (width 0.1) (layer "B.Cu") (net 16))
 (segment (start 147.625 96.496) (end 148.631 97.502) (width 0.1) (layer "F.Cu") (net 7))
 (segment (start 134.8 98.697288) (end 137.001288 96.496) (width 0.1) (layer "F.Cu") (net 7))
 (segment (start 148.48 102.12) (end 148 102.12) (width 0.1) (layer "F.Cu") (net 7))
 (segment (start 137.001288 96.496) (end 147.625 96.496) (width 0.1) (layer "F.Cu") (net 7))
 (segment (start 148.631 97.502) (end 148.631 101.969) (width 0.1) (layer "F.Cu") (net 7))
 (segment (start 148.631 101.969) (end 148.48 102.12) (width 0.1) (layer "F.Cu") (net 7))
 (segment (start 134.8 103.3) (end 134.8 98.697288) (width 0.1) (layer "F.Cu") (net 7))
 (segment (start 150.437 96.411322) (end 150.437 103.955) (width 0.1) (layer "F.Cu") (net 19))
 (segment (start 135.7 93.6) (end 147.625678 93.6) (width 0.1) (layer "F.Cu") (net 19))
 (segment (start 148.432 105.96) (end 148 105.96) (width 0.1) (layer "F.Cu") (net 19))
 (segment (start 147.625678 93.6) (end 150.437 96.411322) (width 0.1) (layer "F.Cu") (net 19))
 (segment (start 150.437 103.955) (end 148.432 105.96) (width 0.1) (layer "F.Cu") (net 19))
 (via (at 135.7 93.6) (size 0.6) (drill 0.3) (layers "F.Cu" "B.Cu") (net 19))
 (segment (start 135.649 93.651) (end 135.7 93.6) (width 0.1) (layer "B.Cu") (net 19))
 (segment (start 135.649 94.528232) (end 135.649 93.651) (width 0.1) (layer "B.Cu") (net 19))
 (segment (start 135.8 94.679232) (end 135.649 94.528232) (width 0.1) (layer "B.Cu") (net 19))
 (segment (start 135.8 103.3) (end 135.8 94.679232) (width 0.1) (layer "B.Cu") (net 19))
 (segment (start 149.233 97.252644) (end 149.233 102.647) (width 0.1) (layer "F.Cu") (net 5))
 (segment (start 147.874356 95.894) (end 149.233 97.252644) (width 0.1) (layer "F.Cu") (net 5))
 (segment (start 149.233 102.647) (end 148.48 103.4) (width 0.1) (layer "F.Cu") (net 5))
 (segment (start 136.751932 95.894) (end 147.874356 95.894) (width 0.1) (layer "F.Cu") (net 5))
 (segment (start 148.48 103.4) (end 148 103.4) (width 0.1) (layer "F.Cu") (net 5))
 (segment (start 133.8 98.845932) (end 136.751932 95.894) (width 0.1) (layer "F.Cu") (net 5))
 (segment (start 133.8 103.3) (end 133.8 98.845932) (width 0.1) (layer "F.Cu") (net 5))
 (segment (start 136.8 94.9) (end 148.048678 94.9) (width 0.1) (layer "F.Cu") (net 21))
 (segment (start 149.835 96.686322) (end 149.835 103.277) (width 0.1) (layer "F.Cu") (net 21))
 (segment (start 148.432 104.68) (end 148 104.68) (width 0.1) (layer "F.Cu") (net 21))
 (segment (start 148.048678 94.9) (end 149.835 96.686322) (width 0.1) (layer "F.Cu") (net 21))
 (segment (start 149.835 103.277) (end 148.432 104.68) (width 0.1) (layer "F.Cu") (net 21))
 (via (at 136.8 94.9) (size 0.6) (drill 0.3) (layers "F.Cu" "B.Cu") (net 21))
 (segment (start 136.8 103.3) (end 136.8 94.9) (width 0.1) (layer "B.Cu") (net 21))
 (segment (start 144.174356 97.098) (end 145.237 98.160644) (width 0.1) (layer "F.Cu") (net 9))
 (segment (start 137.250644 97.098) (end 144.174356 97.098) (width 0.1) (layer "F.Cu") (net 9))
 (segment (start 145.237 98.160644) (end 145.237 102.512) (width 0.1) (layer "F.Cu") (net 9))
 (segment (start 145.237 102.512) (end 145.455 102.73) (width 0.1) (layer "F.Cu") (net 9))
 (segment (start 145.455 102.73) (end 147.03 102.73) (width 0.1) (layer "F.Cu") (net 9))
 (segment (start 147.03 102.73) (end 147.06 102.76) (width 0.1) (layer "F.Cu") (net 9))
 (segment (start 135.8 103.3) (end 135.8 98.548644) (width 0.1) (layer "F.Cu") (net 9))
 (segment (start 135.8 98.548644) (end 137.250644 97.098) (width 0.1) (layer "F.Cu") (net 9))
 (segment (start 148.932 97.377322) (end 148.932 102.308) (width 0.1) (layer "F.Cu") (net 6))
 (segment (start 147.749678 96.195) (end 148.932 97.377322) (width 0.1) (layer "F.Cu") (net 6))
 (segment (start 148.932 102.308) (end 148.48 102.76) (width 0.1) (layer "F.Cu") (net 6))
 (segment (start 136.87661 96.195) (end 147.749678 96.195) (width 0.1) (layer "F.Cu") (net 6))
 (segment (start 148.48 102.76) (end 148 102.76) (width 0.1) (layer "F.Cu") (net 6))
 (segment (start 134.3 103.3) (end 134.3 98.77161) (width 0.1) (layer "F.Cu") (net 6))
 (segment (start 134.3 98.77161) (end 136.87661 96.195) (width 0.1) (layer "F.Cu") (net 6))
 (segment (start 146.285 104.71) (end 147.03 104.71) (width 0.1) (layer "F.Cu") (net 14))
 (segment (start 147.03 104.71) (end 147.06 104.68) (width 0.1) (layer "F.Cu") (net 14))
 (via (at 146.285 104.71) (size 0.6) (drill 0.3) (layers "F.Cu" "B.Cu") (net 14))
 (segment (start 133.3 91.425678) (end 133.824678 90.901) (width 0.1) (layer "B.Cu") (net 14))
 (segment (start 133.824678 90.901) (end 138.752843 90.901) (width 0.1) (layer "B.Cu") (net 14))
 (segment (start 146.285 98.433157) (end 146.285 104.71) (width 0.1) (layer "B.Cu") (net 14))
 (segment (start 133.3 103.3) (end 133.3 91.425678) (width 0.1) (layer "B.Cu") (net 14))
 (segment (start 138.752843 90.901) (end 146.285 98.433157) (width 0.1) (layer "B.Cu") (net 14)))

